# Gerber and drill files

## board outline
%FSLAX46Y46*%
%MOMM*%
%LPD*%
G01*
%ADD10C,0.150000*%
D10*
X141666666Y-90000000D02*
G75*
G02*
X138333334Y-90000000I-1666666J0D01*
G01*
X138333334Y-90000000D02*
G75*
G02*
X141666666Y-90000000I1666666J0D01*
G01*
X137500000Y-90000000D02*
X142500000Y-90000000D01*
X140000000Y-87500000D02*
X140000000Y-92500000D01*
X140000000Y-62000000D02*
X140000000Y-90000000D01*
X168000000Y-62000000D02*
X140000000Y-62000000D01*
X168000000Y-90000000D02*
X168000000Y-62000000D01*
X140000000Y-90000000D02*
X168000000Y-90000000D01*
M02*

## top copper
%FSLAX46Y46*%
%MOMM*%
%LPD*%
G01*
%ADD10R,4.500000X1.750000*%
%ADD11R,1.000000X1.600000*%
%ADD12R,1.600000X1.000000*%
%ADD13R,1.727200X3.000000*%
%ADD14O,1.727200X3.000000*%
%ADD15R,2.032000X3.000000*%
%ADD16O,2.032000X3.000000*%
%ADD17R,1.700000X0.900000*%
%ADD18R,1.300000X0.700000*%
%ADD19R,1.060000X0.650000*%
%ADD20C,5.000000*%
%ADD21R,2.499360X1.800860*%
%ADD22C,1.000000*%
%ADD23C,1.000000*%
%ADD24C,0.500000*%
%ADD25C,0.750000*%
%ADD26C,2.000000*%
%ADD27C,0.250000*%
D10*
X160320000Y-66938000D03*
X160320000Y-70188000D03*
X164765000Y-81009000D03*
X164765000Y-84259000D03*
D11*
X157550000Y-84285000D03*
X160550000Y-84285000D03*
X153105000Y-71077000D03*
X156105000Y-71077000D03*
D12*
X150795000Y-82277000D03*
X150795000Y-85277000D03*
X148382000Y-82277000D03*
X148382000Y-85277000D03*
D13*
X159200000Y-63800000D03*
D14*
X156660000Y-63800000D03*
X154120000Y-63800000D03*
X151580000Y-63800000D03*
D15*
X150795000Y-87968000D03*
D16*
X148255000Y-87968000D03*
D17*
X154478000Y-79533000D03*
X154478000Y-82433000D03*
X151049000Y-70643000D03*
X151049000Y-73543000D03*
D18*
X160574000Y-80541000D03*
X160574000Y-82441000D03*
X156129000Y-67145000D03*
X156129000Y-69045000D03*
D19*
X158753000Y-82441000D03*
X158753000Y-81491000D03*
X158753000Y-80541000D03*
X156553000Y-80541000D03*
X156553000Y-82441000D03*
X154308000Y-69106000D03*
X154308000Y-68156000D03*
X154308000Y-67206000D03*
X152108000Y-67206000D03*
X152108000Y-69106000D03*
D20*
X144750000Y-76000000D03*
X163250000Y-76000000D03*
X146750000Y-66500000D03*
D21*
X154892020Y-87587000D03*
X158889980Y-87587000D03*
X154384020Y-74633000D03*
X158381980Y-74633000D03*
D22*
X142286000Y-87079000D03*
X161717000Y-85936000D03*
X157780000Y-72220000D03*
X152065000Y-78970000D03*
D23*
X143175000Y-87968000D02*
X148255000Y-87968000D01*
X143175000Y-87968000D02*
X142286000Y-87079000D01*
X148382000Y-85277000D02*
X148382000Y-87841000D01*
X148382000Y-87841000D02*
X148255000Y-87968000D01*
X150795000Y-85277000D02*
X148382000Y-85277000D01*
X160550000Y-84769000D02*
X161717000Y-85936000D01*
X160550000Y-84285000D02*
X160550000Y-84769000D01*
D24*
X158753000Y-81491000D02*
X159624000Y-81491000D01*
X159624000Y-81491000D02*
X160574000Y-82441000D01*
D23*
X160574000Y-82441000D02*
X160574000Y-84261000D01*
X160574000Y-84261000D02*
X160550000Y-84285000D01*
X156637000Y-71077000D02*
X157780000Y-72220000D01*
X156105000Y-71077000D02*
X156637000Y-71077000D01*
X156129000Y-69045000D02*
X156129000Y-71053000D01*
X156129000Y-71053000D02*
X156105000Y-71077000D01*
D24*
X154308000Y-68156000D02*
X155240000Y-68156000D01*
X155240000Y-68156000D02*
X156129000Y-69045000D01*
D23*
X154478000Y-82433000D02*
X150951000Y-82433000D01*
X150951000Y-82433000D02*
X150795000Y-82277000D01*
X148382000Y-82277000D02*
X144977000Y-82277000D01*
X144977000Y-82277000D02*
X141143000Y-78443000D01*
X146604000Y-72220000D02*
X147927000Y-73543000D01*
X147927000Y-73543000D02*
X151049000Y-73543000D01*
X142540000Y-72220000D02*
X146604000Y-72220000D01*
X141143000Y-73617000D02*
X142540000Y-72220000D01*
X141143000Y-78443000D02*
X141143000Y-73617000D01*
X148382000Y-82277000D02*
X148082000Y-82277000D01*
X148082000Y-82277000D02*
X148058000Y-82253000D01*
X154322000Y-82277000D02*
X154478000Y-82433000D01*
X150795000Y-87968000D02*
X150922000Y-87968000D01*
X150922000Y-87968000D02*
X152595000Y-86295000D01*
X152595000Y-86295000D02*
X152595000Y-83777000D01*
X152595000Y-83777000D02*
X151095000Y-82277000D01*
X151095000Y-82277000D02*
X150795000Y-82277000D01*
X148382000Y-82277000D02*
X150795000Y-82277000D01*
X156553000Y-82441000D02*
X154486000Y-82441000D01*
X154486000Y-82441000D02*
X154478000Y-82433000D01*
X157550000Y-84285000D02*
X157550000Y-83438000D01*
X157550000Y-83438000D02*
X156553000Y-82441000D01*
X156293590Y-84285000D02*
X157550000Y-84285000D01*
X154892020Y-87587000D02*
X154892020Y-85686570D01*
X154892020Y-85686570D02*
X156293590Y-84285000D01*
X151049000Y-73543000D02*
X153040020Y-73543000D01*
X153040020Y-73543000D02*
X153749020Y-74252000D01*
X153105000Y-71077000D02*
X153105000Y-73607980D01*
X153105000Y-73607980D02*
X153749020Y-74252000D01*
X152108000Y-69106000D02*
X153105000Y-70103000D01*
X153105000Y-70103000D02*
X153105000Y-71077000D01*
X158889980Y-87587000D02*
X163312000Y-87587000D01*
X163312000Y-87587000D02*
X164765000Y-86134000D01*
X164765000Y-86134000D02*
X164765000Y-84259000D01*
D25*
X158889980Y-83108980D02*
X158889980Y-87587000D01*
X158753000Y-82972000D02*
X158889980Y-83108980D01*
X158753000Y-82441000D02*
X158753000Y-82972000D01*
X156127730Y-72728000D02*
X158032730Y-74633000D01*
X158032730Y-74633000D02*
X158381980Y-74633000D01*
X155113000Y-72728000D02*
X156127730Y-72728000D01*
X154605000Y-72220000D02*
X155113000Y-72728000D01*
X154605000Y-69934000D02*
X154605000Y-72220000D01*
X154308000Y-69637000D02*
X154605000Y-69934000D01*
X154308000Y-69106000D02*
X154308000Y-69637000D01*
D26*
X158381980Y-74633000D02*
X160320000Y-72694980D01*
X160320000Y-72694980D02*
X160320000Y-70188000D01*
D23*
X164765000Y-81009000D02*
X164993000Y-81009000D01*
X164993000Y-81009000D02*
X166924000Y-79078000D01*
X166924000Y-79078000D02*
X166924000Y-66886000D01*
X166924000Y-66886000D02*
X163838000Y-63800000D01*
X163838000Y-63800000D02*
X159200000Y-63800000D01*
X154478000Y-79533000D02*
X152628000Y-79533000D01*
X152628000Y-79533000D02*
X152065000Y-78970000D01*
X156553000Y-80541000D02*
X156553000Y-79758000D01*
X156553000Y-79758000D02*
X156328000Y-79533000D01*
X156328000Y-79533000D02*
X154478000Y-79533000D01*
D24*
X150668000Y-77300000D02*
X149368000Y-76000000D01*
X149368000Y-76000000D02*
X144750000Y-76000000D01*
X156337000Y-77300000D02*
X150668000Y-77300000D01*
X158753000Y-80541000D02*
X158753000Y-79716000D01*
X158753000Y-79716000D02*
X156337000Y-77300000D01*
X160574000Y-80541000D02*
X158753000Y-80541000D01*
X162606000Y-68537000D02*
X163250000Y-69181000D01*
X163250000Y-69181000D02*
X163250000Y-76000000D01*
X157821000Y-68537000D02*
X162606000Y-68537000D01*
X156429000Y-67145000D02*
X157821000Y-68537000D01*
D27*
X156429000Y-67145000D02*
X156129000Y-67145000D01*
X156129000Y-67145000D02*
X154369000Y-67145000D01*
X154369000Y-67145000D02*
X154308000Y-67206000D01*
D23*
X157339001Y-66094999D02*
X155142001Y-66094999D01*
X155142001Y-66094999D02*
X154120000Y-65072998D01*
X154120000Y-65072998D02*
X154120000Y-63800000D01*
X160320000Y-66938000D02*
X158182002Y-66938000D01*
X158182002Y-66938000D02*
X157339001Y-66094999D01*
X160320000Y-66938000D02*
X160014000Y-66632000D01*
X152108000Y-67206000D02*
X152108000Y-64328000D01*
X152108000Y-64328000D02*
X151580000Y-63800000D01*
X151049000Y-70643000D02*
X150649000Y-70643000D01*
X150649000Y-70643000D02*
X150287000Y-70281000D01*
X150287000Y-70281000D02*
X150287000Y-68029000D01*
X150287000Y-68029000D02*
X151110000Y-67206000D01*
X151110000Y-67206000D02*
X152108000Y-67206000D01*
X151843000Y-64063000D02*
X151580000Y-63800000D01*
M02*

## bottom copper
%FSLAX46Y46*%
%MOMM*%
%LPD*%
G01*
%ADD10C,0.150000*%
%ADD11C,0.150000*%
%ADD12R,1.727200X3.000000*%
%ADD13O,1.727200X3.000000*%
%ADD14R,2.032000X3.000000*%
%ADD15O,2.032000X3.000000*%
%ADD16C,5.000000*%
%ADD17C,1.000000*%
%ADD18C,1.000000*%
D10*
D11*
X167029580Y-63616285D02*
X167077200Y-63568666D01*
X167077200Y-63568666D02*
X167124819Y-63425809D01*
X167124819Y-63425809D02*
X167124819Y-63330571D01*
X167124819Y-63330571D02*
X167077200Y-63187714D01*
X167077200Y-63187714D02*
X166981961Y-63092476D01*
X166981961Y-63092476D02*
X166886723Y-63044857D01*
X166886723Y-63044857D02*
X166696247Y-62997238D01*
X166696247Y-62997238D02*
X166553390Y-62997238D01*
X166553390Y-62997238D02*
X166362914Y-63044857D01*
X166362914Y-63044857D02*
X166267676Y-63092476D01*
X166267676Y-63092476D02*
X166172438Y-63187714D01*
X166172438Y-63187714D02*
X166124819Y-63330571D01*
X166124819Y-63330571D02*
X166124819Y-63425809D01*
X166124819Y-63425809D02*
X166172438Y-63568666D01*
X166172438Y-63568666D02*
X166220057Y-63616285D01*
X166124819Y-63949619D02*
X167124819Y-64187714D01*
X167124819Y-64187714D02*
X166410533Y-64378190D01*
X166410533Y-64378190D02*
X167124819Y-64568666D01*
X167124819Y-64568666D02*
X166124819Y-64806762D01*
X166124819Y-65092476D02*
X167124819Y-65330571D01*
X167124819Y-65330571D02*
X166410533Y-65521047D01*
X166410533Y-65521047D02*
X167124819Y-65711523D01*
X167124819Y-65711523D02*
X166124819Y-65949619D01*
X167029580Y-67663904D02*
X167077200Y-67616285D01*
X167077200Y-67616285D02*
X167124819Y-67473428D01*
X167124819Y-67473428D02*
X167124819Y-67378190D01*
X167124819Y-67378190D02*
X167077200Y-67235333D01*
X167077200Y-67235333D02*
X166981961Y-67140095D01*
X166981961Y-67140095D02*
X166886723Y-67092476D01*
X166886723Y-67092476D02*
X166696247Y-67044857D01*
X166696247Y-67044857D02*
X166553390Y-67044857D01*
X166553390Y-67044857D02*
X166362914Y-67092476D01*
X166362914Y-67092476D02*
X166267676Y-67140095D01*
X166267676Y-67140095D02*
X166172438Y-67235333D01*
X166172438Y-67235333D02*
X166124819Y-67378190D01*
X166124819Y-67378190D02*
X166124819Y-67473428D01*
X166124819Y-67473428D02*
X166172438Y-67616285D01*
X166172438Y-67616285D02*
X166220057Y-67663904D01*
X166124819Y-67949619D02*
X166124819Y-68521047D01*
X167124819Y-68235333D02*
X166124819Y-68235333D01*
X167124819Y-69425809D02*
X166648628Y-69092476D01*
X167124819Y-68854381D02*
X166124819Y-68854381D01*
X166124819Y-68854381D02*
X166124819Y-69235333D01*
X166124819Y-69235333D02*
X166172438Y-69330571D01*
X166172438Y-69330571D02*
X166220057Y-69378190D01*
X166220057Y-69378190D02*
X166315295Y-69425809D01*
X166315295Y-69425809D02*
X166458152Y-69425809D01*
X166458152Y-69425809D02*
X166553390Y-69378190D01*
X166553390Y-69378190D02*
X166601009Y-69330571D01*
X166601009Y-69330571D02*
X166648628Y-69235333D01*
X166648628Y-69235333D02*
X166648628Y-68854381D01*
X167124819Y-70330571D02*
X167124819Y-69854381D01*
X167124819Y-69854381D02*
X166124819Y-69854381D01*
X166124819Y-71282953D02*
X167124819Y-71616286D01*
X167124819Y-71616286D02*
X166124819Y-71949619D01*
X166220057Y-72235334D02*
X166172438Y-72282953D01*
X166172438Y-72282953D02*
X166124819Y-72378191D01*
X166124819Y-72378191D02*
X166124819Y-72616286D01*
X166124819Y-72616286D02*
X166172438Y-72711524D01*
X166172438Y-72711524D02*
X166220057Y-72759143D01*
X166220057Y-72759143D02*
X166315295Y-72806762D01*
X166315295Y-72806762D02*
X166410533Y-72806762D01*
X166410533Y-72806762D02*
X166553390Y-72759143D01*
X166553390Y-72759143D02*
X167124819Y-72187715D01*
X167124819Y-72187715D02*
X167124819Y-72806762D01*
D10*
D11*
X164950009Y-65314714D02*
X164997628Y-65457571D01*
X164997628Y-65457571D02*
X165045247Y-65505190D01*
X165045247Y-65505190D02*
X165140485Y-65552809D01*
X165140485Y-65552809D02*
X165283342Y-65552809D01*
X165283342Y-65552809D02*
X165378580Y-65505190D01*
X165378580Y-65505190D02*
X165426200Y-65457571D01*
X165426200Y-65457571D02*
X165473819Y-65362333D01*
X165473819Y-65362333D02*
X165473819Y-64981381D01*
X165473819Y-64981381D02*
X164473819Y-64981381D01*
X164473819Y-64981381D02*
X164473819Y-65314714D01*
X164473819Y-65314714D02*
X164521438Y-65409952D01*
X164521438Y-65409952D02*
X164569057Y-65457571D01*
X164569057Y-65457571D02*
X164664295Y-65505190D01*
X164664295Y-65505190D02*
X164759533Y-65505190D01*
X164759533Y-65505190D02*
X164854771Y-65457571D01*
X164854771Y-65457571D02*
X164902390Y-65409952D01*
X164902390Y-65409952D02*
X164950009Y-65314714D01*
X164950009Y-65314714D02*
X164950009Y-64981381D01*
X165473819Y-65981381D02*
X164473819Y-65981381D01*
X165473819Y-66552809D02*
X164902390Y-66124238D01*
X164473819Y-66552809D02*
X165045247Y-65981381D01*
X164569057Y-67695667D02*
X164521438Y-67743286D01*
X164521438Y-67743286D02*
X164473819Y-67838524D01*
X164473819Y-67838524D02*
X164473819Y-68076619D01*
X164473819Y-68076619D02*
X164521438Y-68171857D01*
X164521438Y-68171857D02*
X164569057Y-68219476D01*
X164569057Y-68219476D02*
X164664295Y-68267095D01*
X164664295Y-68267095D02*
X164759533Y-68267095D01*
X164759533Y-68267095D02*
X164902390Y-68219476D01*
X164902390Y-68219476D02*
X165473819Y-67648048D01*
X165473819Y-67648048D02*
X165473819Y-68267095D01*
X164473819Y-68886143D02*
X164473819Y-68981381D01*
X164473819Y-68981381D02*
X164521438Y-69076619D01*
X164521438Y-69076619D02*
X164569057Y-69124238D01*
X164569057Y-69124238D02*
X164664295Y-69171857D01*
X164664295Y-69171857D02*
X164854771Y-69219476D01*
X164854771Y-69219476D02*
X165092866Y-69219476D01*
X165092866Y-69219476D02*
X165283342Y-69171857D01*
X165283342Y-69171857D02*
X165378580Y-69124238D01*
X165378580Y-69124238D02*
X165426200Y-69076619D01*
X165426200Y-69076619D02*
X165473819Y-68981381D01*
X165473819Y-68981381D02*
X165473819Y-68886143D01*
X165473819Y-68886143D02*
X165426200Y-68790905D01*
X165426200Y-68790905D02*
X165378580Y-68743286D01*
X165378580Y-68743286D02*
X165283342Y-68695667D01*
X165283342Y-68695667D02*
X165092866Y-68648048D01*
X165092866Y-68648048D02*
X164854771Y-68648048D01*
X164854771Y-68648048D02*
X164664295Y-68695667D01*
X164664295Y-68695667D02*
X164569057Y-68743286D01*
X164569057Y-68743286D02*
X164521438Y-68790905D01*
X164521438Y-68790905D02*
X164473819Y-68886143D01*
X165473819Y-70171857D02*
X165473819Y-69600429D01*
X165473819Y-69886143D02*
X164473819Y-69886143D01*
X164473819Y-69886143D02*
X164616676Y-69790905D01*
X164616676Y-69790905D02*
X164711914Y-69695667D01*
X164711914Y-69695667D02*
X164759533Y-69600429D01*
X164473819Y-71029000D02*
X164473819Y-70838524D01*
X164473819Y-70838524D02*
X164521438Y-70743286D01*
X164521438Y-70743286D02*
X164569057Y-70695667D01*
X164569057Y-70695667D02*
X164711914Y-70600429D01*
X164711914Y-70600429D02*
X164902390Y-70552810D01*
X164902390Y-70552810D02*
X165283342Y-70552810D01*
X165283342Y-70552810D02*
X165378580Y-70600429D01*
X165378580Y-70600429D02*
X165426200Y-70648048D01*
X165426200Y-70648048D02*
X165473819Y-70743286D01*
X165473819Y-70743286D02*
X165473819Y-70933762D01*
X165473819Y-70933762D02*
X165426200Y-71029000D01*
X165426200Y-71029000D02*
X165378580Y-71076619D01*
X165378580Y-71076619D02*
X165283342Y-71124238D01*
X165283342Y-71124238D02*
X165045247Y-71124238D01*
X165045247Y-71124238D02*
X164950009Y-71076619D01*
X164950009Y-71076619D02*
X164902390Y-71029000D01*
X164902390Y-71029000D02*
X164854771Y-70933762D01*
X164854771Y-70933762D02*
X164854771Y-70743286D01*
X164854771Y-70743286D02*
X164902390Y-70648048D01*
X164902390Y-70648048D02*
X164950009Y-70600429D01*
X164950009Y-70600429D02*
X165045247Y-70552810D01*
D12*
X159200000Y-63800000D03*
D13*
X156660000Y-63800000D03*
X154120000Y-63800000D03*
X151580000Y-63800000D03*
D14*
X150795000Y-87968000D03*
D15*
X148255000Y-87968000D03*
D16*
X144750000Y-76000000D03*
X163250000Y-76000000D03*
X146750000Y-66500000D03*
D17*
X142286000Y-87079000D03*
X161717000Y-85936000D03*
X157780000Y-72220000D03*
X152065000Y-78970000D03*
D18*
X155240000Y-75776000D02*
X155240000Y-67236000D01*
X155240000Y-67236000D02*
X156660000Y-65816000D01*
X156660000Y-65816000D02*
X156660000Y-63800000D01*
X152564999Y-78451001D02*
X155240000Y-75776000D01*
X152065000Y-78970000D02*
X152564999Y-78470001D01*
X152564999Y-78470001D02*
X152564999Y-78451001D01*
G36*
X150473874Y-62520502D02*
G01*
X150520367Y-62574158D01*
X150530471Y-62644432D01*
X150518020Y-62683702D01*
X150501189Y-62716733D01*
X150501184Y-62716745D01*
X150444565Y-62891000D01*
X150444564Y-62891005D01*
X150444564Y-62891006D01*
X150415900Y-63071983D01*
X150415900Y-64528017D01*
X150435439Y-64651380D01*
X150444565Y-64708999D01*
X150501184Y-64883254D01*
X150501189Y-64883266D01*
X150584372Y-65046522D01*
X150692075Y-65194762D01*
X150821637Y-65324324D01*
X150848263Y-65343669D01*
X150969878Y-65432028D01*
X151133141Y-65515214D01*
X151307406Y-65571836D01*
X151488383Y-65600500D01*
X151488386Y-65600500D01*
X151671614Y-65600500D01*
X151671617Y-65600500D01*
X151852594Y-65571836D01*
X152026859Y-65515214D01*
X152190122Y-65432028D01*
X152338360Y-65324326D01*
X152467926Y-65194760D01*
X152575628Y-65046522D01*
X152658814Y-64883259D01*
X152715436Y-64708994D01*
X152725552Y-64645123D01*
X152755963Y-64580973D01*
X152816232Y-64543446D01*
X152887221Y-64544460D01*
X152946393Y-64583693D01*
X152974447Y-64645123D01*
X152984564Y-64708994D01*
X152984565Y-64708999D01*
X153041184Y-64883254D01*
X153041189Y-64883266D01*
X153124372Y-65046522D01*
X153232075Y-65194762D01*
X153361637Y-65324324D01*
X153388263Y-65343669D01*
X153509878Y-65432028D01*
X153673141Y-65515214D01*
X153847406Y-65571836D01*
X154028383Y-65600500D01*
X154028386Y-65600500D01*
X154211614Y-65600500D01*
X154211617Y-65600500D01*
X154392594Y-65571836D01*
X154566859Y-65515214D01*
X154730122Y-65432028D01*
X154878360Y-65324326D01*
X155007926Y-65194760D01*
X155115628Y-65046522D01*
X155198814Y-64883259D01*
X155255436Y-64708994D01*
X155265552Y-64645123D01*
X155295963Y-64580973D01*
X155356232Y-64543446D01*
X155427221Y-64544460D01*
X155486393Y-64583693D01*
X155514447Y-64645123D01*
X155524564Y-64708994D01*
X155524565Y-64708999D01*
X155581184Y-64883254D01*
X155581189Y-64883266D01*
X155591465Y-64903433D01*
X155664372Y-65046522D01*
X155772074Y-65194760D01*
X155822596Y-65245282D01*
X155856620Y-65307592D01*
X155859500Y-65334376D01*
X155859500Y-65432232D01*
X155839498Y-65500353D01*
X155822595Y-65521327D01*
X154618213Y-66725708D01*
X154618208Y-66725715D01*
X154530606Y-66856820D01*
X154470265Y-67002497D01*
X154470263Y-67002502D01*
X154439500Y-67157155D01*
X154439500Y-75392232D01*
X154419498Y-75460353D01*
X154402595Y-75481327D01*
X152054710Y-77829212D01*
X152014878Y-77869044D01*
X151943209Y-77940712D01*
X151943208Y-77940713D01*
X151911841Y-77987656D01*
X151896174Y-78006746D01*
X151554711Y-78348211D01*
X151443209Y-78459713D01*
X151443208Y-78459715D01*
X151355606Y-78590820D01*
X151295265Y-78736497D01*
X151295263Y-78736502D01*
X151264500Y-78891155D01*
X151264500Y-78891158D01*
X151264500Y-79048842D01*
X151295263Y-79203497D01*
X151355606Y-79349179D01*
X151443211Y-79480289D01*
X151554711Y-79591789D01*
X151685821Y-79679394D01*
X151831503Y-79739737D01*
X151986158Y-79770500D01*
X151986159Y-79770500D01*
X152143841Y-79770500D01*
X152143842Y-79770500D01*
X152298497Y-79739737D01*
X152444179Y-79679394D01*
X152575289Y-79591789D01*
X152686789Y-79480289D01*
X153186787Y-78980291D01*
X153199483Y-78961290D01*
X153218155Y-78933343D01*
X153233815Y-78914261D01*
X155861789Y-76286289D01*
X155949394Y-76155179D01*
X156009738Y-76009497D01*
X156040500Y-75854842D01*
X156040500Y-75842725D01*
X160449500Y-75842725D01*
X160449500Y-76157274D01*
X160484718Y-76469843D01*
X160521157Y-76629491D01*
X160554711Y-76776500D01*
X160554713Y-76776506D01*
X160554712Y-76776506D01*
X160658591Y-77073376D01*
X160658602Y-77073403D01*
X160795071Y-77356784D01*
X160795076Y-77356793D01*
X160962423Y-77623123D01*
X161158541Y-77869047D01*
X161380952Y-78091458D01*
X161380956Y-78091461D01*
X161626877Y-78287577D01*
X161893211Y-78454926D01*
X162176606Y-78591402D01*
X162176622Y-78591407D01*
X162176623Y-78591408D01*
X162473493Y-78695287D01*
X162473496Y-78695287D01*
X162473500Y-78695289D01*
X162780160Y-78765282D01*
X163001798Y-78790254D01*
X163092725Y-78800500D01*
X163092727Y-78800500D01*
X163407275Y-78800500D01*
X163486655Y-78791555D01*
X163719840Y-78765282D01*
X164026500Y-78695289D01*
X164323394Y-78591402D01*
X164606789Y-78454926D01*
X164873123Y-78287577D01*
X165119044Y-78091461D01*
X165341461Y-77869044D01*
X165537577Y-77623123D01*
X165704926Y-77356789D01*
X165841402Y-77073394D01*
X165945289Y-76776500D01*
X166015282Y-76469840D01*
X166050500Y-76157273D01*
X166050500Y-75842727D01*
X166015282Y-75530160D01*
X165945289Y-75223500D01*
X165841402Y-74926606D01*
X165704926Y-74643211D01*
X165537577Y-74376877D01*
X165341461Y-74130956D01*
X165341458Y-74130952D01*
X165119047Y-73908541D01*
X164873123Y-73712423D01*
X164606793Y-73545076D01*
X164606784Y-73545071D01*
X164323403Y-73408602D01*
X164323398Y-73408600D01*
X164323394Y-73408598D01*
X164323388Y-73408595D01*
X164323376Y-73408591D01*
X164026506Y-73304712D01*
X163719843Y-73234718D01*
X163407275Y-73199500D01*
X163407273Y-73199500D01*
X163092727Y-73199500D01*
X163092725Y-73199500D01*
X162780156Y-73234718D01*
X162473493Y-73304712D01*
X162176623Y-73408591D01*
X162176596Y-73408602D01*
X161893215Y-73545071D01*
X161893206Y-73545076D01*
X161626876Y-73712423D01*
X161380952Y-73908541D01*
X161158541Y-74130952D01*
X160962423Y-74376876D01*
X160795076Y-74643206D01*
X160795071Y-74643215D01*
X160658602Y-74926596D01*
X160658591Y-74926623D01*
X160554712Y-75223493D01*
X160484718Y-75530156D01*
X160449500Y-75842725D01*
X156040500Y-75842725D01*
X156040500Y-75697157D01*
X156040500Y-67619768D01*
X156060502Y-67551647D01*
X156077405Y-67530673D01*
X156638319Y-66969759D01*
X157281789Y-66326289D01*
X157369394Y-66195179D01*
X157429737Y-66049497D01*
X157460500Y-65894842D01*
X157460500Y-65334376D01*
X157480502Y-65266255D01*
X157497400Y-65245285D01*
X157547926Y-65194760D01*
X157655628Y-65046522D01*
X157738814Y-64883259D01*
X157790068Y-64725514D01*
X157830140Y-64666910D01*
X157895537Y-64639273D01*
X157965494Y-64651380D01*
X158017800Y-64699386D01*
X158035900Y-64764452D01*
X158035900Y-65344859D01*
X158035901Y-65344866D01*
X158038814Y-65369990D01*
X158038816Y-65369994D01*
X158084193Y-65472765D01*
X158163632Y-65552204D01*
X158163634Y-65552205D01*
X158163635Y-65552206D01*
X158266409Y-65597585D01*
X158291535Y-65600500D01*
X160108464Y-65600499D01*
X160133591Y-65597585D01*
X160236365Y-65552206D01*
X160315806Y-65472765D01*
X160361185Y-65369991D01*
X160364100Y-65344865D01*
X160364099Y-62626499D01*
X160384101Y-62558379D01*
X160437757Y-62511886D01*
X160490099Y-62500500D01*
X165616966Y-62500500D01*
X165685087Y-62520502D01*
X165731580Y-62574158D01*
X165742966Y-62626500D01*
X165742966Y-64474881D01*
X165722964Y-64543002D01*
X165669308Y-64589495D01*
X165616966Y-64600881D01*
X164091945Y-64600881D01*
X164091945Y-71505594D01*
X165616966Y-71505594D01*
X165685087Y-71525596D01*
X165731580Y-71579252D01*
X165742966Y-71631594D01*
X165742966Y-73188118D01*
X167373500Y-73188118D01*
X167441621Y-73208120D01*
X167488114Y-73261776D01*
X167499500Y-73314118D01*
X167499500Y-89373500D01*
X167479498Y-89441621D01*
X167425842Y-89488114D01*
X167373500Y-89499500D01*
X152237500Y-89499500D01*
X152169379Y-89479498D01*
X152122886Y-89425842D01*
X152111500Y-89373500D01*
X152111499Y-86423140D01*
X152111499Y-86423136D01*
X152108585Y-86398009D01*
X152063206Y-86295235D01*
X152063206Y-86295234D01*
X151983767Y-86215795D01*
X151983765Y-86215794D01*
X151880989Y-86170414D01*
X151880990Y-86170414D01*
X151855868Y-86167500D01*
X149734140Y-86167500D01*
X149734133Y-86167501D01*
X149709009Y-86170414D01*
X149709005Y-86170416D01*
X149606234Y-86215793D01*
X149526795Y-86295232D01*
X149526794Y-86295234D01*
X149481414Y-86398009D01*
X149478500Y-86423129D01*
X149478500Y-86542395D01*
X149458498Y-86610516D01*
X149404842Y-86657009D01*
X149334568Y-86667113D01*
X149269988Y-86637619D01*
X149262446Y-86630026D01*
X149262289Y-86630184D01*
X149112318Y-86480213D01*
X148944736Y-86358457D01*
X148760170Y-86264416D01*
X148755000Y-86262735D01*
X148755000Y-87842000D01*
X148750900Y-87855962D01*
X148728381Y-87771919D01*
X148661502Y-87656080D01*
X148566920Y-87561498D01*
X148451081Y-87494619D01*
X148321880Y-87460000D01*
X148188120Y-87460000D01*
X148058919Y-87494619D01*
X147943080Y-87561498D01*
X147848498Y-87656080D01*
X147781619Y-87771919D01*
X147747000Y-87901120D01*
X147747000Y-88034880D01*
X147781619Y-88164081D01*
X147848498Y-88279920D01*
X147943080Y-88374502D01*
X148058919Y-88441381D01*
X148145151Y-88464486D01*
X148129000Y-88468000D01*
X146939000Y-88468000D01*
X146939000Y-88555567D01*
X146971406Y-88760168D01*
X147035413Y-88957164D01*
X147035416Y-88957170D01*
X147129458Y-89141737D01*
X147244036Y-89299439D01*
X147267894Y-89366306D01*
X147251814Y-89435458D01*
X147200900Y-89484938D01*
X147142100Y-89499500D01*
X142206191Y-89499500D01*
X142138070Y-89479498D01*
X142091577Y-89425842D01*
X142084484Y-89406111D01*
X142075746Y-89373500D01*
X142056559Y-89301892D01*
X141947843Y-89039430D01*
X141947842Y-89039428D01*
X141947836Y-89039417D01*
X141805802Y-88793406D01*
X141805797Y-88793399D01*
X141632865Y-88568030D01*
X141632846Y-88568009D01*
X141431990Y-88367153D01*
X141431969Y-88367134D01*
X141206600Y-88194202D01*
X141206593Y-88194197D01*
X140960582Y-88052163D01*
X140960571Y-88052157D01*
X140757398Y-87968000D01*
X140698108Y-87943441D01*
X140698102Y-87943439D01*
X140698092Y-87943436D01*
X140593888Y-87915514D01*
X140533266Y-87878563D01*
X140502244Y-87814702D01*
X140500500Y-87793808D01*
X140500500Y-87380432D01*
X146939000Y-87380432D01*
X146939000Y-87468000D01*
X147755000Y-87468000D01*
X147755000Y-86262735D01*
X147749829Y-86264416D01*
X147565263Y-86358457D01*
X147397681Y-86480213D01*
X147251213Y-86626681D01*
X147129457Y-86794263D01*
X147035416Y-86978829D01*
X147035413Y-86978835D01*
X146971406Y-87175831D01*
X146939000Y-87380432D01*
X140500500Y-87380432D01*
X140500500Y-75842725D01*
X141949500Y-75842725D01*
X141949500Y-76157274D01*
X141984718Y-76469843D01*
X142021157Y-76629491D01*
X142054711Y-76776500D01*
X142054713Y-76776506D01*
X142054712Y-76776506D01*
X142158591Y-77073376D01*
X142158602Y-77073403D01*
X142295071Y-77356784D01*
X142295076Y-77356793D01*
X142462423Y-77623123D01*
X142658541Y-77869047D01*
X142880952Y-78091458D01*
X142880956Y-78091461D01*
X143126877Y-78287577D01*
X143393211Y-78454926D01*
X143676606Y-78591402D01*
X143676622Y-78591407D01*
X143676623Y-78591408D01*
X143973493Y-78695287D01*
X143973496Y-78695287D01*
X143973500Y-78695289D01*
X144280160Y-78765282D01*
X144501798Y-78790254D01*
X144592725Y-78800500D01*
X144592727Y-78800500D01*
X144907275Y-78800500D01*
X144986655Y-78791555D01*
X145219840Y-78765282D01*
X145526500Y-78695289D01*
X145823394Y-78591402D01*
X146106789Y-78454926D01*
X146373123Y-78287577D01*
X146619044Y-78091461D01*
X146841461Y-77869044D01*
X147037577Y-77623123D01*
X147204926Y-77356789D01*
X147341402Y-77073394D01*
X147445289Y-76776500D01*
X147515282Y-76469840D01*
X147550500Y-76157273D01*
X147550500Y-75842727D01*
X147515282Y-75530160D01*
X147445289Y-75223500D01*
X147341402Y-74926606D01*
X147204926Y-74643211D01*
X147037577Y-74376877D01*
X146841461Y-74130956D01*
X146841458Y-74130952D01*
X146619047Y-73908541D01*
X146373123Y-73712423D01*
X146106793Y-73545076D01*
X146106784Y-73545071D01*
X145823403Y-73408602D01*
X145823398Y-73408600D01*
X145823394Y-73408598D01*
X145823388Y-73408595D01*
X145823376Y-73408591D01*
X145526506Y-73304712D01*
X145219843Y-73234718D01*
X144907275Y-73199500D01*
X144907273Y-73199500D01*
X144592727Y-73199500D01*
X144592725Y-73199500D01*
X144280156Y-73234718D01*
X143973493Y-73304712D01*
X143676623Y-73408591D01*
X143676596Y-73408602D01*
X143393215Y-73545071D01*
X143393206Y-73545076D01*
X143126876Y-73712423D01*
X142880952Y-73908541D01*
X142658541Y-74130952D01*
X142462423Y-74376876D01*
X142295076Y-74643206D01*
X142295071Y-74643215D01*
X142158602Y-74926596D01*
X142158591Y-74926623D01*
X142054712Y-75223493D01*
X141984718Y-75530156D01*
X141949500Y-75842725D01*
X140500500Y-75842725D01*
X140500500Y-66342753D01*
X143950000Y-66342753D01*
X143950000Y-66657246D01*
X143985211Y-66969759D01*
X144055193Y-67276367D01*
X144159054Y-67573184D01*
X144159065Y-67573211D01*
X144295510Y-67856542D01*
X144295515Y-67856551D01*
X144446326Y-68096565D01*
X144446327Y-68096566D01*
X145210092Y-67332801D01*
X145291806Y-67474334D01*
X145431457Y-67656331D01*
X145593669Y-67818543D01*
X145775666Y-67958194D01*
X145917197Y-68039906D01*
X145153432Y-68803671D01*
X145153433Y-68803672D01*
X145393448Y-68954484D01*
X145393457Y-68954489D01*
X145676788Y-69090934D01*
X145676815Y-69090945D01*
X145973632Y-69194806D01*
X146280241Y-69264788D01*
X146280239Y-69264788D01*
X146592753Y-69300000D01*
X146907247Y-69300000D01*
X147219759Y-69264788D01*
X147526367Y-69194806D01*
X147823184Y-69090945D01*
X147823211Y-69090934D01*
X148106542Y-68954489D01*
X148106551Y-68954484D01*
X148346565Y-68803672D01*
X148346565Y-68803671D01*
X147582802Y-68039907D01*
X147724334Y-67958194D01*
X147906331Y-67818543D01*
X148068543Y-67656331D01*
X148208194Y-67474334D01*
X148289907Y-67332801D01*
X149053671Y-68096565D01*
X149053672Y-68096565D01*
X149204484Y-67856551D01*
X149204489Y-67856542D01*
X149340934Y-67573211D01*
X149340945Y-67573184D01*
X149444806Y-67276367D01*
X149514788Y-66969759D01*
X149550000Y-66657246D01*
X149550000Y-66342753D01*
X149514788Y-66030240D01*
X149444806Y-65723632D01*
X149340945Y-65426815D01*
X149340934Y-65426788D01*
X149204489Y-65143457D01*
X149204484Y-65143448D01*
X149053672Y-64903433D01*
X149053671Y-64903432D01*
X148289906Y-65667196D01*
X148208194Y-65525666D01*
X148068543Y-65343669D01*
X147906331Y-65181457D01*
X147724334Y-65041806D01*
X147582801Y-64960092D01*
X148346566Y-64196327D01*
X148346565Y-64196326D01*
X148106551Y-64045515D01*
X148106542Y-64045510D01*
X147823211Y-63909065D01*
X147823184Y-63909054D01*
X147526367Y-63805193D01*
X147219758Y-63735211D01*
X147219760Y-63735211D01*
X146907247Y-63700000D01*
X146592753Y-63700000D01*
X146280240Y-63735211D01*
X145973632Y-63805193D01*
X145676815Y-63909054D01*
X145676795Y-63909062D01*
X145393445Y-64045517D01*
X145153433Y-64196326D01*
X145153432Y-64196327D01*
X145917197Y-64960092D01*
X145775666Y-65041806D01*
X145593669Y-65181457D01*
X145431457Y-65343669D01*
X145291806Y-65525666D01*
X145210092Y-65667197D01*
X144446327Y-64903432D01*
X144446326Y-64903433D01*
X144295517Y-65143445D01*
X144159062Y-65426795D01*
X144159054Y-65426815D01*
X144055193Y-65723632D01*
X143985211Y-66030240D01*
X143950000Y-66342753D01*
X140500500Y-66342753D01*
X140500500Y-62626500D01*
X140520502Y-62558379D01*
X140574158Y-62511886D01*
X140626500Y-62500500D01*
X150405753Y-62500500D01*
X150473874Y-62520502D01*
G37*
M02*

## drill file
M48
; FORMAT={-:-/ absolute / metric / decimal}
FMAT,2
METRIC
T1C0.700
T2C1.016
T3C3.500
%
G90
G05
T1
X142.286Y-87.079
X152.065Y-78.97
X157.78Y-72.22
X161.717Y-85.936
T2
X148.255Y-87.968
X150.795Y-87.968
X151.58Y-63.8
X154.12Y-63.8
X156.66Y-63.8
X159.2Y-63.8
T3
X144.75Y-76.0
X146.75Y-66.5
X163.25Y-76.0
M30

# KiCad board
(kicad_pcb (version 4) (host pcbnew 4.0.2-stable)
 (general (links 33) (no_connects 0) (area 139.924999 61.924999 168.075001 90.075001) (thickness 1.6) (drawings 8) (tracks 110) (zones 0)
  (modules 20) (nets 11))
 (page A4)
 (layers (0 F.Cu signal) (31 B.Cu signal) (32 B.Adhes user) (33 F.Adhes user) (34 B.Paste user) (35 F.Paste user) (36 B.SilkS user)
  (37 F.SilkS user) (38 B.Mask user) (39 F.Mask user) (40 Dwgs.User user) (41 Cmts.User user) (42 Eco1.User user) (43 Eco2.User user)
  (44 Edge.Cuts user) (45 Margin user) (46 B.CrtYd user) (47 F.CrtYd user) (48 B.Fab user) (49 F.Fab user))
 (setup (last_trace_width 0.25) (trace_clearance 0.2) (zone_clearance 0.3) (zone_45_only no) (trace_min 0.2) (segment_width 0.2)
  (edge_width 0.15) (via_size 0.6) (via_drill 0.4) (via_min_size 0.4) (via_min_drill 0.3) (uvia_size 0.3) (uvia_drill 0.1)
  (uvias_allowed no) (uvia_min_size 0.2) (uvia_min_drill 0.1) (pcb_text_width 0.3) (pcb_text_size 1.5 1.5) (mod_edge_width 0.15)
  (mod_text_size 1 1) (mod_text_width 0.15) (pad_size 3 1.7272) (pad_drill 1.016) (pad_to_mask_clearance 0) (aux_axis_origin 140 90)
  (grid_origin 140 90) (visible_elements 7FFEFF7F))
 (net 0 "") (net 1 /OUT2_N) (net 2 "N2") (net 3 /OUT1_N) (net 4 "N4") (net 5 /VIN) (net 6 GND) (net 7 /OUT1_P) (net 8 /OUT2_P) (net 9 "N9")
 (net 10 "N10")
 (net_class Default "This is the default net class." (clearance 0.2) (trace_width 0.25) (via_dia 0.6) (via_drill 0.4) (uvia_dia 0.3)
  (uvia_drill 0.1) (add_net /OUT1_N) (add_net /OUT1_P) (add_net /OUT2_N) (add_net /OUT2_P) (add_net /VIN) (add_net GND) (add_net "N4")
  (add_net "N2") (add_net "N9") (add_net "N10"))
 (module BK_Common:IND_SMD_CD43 (layer F.Cu) (at 160.32 68.563 270)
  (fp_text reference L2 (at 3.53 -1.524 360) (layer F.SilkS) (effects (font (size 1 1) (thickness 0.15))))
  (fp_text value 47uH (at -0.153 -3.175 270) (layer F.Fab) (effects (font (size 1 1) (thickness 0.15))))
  (pad 1 smd rect (at -1.625 0 270) (size 1.75 4.5) (layers F.Cu F.Paste F.Mask) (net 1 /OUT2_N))
  (pad 2 smd rect (at 1.625 0 270) (size 1.75 4.5) (layers F.Cu F.Paste F.Mask) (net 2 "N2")))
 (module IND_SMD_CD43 (layer F.Cu) (at 164.765 82.634 270)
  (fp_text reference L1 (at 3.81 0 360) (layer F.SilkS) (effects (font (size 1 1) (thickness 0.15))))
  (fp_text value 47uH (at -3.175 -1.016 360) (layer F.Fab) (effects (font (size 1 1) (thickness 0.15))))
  (pad 1 smd rect (at -1.625 0 270) (size 1.75 4.5) (layers F.Cu F.Paste F.Mask) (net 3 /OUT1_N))
  (pad 2 smd rect (at 1.625 0 270) (size 1.75 4.5) (layers F.Cu F.Paste F.Mask) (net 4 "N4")))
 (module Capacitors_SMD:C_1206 (layer F.Cu) (at 159.05 84.285)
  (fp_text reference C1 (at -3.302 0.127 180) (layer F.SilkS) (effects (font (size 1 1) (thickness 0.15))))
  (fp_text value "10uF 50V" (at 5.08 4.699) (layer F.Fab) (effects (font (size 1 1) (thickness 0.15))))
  (pad 1 smd rect (at -1.5 0) (size 1 1.6) (layers F.Cu F.Paste F.Mask) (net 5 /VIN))
  (pad 2 smd rect (at 1.5 0) (size 1 1.6) (layers F.Cu F.Paste F.Mask) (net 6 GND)))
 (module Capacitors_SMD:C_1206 (layer F.Cu) (at 154.605 71.077)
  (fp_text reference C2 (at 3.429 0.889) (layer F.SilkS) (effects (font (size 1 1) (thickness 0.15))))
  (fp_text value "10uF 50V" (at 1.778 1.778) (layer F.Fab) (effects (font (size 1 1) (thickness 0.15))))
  (pad 1 smd rect (at -1.5 0) (size 1 1.6) (layers F.Cu F.Paste F.Mask) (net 5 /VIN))
  (pad 2 smd rect (at 1.5 0) (size 1 1.6) (layers F.Cu F.Paste F.Mask) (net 6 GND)))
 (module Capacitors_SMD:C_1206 (layer F.Cu) (at 150.795 83.777 270)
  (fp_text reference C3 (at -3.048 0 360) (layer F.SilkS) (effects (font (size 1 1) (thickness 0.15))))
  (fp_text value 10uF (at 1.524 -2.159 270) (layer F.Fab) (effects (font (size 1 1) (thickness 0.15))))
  (pad 1 smd rect (at -1.5 0 270) (size 1 1.6) (layers F.Cu F.Paste F.Mask) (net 5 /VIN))
  (pad 2 smd rect (at 1.5 0 270) (size 1 1.6) (layers F.Cu F.Paste F.Mask) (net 6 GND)))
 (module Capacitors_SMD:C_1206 (layer F.Cu) (at 148.382 83.777 270)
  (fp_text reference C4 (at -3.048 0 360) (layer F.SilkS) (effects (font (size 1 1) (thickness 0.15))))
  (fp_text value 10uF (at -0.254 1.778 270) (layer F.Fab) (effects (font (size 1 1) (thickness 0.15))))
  (pad 1 smd rect (at -1.5 0 270) (size 1 1.6) (layers F.Cu F.Paste F.Mask) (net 5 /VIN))
  (pad 2 smd rect (at 1.5 0 270) (size 1 1.6) (layers F.Cu F.Paste F.Mask) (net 6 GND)))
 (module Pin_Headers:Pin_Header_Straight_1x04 (layer F.Cu) (at 159.2 63.8 270)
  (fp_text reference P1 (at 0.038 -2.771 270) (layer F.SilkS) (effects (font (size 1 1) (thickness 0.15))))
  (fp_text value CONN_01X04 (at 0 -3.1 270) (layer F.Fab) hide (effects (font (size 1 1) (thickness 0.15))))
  (pad 1 thru_hole rect (at 0 0 270) (size 3 1.7272) (drill 1.016) (layers *.Cu *.Mask F.SilkS) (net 3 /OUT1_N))
  (pad 2 thru_hole oval (at 0 2.54 270) (size 3 1.7272) (drill 1.016) (layers *.Cu *.Mask F.SilkS) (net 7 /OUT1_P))
  (pad 3 thru_hole oval (at 0 5.08 270) (size 3 1.7272) (drill 1.016) (layers *.Cu *.Mask F.SilkS) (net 1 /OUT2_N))
  (pad 4 thru_hole oval (at 0 7.62 270) (size 3 1.7272) (drill 1.016) (layers *.Cu *.Mask F.SilkS) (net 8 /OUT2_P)))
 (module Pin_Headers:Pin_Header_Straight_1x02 (layer F.Cu) (at 150.795 87.968 270)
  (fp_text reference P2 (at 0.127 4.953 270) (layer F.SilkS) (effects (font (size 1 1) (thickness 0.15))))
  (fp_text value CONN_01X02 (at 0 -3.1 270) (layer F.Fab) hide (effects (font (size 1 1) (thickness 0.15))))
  (pad 1 thru_hole rect (at 0 0 270) (size 3 2.032) (drill 1.016) (layers *.Cu *.Mask F.SilkS) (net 5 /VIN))
  (pad 2 thru_hole oval (at 0 2.54 270) (size 3 2.032) (drill 1.016) (layers *.Cu *.Mask F.SilkS) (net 6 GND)))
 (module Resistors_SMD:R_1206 (layer F.Cu) (at 154.478 80.983 270)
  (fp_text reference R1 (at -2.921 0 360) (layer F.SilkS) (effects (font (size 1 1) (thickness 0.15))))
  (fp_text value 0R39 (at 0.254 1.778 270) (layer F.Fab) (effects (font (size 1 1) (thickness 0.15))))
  (pad 1 smd rect (at -1.45 0 270) (size 0.9 1.7) (layers F.Cu F.Paste F.Mask) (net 7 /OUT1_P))
  (pad 2 smd rect (at 1.45 0 270) (size 0.9 1.7) (layers F.Cu F.Paste F.Mask) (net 5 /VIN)))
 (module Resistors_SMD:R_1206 (layer F.Cu) (at 151.049 72.093 270)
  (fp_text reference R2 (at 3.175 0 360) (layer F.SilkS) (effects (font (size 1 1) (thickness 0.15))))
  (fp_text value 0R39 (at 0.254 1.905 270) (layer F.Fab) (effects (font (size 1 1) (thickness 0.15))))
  (pad 1 smd rect (at -1.45 0 270) (size 0.9 1.7) (layers F.Cu F.Paste F.Mask) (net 8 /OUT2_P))
  (pad 2 smd rect (at 1.45 0 270) (size 0.9 1.7) (layers F.Cu F.Paste F.Mask) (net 5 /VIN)))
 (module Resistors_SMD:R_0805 (layer F.Cu) (at 160.574 81.491 270)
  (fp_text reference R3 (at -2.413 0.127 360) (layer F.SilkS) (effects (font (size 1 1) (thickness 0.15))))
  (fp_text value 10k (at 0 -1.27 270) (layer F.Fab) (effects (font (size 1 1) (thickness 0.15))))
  (pad 1 smd rect (at -0.95 0 270) (size 0.7 1.3) (layers F.Cu F.Paste F.Mask) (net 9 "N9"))
  (pad 2 smd rect (at 0.95 0 270) (size 0.7 1.3) (layers F.Cu F.Paste F.Mask) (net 6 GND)))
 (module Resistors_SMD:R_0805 (layer F.Cu) (at 156.129 68.095 270)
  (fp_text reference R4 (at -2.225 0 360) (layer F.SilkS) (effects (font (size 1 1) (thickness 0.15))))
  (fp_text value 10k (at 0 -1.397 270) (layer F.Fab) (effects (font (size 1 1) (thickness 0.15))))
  (pad 1 smd rect (at -0.95 0 270) (size 0.7 1.3) (layers F.Cu F.Paste F.Mask) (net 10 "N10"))
  (pad 2 smd rect (at 0.95 0 270) (size 0.7 1.3) (layers F.Cu F.Paste F.Mask) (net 6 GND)))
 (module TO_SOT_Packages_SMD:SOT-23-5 (layer F.Cu) (at 157.653 81.491 180)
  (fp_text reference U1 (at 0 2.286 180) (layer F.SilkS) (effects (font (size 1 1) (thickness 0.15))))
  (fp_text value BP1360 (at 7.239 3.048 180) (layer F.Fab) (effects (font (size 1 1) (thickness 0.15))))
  (pad 1 smd rect (at -1.1 -0.95 180) (size 1.06 0.65) (layers F.Cu F.Paste F.Mask) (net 4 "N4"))
  (pad 2 smd rect (at -1.1 0 180) (size 1.06 0.65) (layers F.Cu F.Paste F.Mask) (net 6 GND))
  (pad 3 smd rect (at -1.1 0.95 180) (size 1.06 0.65) (layers F.Cu F.Paste F.Mask) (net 9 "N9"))
  (pad 4 smd rect (at 1.1 0.95 180) (size 1.06 0.65) (layers F.Cu F.Paste F.Mask) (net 7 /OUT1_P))
  (pad 5 smd rect (at 1.1 -0.95 180) (size 1.06 0.65) (layers F.Cu F.Paste F.Mask) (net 5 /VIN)))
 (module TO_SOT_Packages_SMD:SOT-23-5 (layer F.Cu) (at 153.208 68.156 180)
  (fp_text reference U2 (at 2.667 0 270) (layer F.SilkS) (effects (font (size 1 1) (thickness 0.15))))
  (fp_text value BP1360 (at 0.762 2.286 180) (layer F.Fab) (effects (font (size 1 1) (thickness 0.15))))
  (pad 1 smd rect (at -1.1 -0.95 180) (size 1.06 0.65) (layers F.Cu F.Paste F.Mask) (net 2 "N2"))
  (pad 2 smd rect (at -1.1 0 180) (size 1.06 0.65) (layers F.Cu F.Paste F.Mask) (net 6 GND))
  (pad 3 smd rect (at -1.1 0.95 180) (size 1.06 0.65) (layers F.Cu F.Paste F.Mask) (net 10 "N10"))
  (pad 4 smd rect (at 1.1 0.95 180) (size 1.06 0.65) (layers F.Cu F.Paste F.Mask) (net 8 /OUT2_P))
  (pad 5 smd rect (at 1.1 -0.95 180) (size 1.06 0.65) (layers F.Cu F.Paste F.Mask) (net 5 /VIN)))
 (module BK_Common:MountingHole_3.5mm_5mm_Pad (layer F.Cu) (at 144.75 76)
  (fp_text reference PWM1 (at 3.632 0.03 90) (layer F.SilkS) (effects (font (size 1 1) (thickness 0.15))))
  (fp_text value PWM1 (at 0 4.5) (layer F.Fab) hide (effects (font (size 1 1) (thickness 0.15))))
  (pad 1 thru_hole circle (at 0 0) (size 5 5) (drill 3.5) (layers *.Cu *.Mask F.SilkS) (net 9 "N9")))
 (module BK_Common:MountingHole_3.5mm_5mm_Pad (layer F.Cu) (at 163.25 76)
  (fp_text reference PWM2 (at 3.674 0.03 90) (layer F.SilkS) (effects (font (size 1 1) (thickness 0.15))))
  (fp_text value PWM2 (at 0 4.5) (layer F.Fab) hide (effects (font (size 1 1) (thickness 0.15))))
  (pad 1 thru_hole circle (at 0 0) (size 5 5) (drill 3.5) (layers *.Cu *.Mask F.SilkS) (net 10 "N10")))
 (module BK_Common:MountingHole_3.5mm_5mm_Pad (layer F.Cu) (at 146.75 66.5)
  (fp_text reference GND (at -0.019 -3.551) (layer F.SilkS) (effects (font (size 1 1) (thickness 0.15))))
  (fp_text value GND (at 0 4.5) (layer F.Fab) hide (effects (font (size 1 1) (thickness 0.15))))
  (pad 1 thru_hole circle (at 0 0) (size 5 5) (drill 3.5) (layers *.Cu *.Mask F.SilkS) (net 6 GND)))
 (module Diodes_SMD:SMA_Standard (layer F.Cu) (at 156.891 87.587)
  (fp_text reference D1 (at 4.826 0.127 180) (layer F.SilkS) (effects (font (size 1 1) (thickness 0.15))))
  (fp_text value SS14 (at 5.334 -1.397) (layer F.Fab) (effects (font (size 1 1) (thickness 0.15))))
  (pad 1 smd rect (at -1.99898 0) (size 2.49936 1.80086) (layers F.Cu F.Paste F.Mask) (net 5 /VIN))
  (pad 2 smd rect (at 1.99898 0) (size 2.49936 1.80086) (layers F.Cu F.Paste F.Mask) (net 4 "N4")))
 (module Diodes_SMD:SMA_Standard (layer F.Cu) (at 156.383 74.633)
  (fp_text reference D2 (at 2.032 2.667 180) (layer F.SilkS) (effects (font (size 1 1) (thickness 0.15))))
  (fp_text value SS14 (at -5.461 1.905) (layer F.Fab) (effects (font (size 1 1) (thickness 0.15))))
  (pad 1 smd rect (at -1.99898 0) (size 2.49936 1.80086) (layers F.Cu F.Paste F.Mask) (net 5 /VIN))
  (pad 2 smd rect (at 1.99898 0) (size 2.49936 1.80086) (layers F.Cu F.Paste F.Mask) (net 2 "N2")))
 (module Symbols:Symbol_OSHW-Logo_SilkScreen (layer F.Cu) (at 143.556 81.999)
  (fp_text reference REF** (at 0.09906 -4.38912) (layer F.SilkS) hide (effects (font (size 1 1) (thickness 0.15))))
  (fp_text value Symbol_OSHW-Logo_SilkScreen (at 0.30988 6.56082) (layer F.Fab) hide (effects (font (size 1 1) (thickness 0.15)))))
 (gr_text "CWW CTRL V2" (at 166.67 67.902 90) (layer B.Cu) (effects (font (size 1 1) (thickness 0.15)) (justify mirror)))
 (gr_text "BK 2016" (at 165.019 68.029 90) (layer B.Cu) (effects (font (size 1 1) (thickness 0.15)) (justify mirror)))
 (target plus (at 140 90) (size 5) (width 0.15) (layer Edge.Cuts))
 (gr_line (start 140 62) (end 140 90) (layer Edge.Cuts) (width 0.15))
 (gr_line (start 168 62) (end 140 62) (layer Edge.Cuts) (width 0.15))
 (gr_line (start 168 90) (end 168 62) (layer Edge.Cuts) (width 0.15))
 (gr_line (start 140 90) (end 168 90) (layer Edge.Cuts) (width 0.15))
 (segment (start 143.175 87.968) (end 148.255 87.968) (width 1) (layer F.Cu) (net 6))
 (via (at 142.286 87.079) (size 1) (drill 0.7) (layers F.Cu B.Cu) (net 6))
 (segment (start 143.175 87.968) (end 142.286 87.079) (width 1) (layer F.Cu) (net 6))
 (segment (start 148.382 85.277) (end 148.382 87.841) (width 1) (layer F.Cu) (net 6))
 (segment (start 148.382 87.841) (end 148.255 87.968) (width 1) (layer F.Cu) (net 6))
 (segment (start 150.795 85.277) (end 148.382 85.277) (width 1) (layer F.Cu) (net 6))
 (via (at 161.717 85.936) (size 1) (drill 0.7) (layers F.Cu B.Cu) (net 6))
 (segment (start 160.55 84.769) (end 161.717 85.936) (width 1) (layer F.Cu) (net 6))
 (segment (start 160.55 84.285) (end 160.55 84.769) (width 1) (layer F.Cu) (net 6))
 (segment (start 158.753 81.491) (end 159.624 81.491) (width 0.5) (layer F.Cu) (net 6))
 (segment (start 159.624 81.491) (end 160.574 82.441) (width 0.5) (layer F.Cu) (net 6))
 (segment (start 160.574 82.441) (end 160.574 84.261) (width 1) (layer F.Cu) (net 6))
 (segment (start 160.574 84.261) (end 160.55 84.285) (width 1) (layer F.Cu) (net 6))
 (via (at 157.78 72.22) (size 1) (drill 0.7) (layers F.Cu B.Cu) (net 6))
 (segment (start 156.637 71.077) (end 157.78 72.22) (width 1) (layer F.Cu) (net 6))
 (segment (start 156.105 71.077) (end 156.637 71.077) (width 1) (layer F.Cu) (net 6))
 (segment (start 156.129 69.045) (end 156.129 71.053) (width 1) (layer F.Cu) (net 6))
 (segment (start 156.129 71.053) (end 156.105 71.077) (width 1) (layer F.Cu) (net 6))
 (segment (start 154.308 68.156) (end 155.24 68.156) (width 0.5) (layer F.Cu) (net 6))
 (segment (start 155.24 68.156) (end 156.129 69.045) (width 0.5) (layer F.Cu) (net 6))
 (segment (start 154.478 82.433) (end 150.951 82.433) (width 1) (layer F.Cu) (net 5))
 (segment (start 150.951 82.433) (end 150.795 82.277) (width 1) (layer F.Cu) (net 5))
 (segment (start 148.382 82.277) (end 144.977 82.277) (width 1) (layer F.Cu) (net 5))
 (segment (start 144.977 82.277) (end 141.143 78.443) (width 1) (layer F.Cu) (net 5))
 (segment (start 146.604 72.22) (end 147.927 73.543) (width 1) (layer F.Cu) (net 5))
 (segment (start 147.927 73.543) (end 151.049 73.543) (width 1) (layer F.Cu) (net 5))
 (segment (start 142.54 72.22) (end 146.604 72.22) (width 1) (layer F.Cu) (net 5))
 (segment (start 141.143 73.617) (end 142.54 72.22) (width 1) (layer F.Cu) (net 5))
 (segment (start 141.143 78.443) (end 141.143 73.617) (width 1) (layer F.Cu) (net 5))
 (segment (start 148.382 82.277) (end 148.082 82.277) (width 1) (layer F.Cu) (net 5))
 (segment (start 148.082 82.277) (end 148.058 82.253) (width 1) (layer F.Cu) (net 5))
 (segment (start 154.322 82.277) (end 154.478 82.433) (width 1) (layer F.Cu) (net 5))
 (segment (start 150.795 87.968) (end 150.922 87.968) (width 1) (layer F.Cu) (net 5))
 (segment (start 150.922 87.968) (end 152.595 86.295) (width 1) (layer F.Cu) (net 5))
 (segment (start 152.595 86.295) (end 152.595 83.777) (width 1) (layer F.Cu) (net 5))
 (segment (start 152.595 83.777) (end 151.095 82.277) (width 1) (layer F.Cu) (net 5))
 (segment (start 151.095 82.277) (end 150.795 82.277) (width 1) (layer F.Cu) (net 5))
 (segment (start 148.382 82.277) (end 150.795 82.277) (width 1) (layer F.Cu) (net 5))
 (segment (start 156.553 82.441) (end 154.486 82.441) (width 1) (layer F.Cu) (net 5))
 (segment (start 154.486 82.441) (end 154.478 82.433) (width 1) (layer F.Cu) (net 5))
 (segment (start 157.55 84.285) (end 157.55 83.438) (width 1) (layer F.Cu) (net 5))
 (segment (start 157.55 83.438) (end 156.553 82.441) (width 1) (layer F.Cu) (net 5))
 (segment (start 156.29359 84.285) (end 157.55 84.285) (width 1) (layer F.Cu) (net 5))
 (segment (start 154.89202 87.587) (end 154.89202 85.68657) (width 1) (layer F.Cu) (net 5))
 (segment (start 154.89202 85.68657) (end 156.29359 84.285) (width 1) (layer F.Cu) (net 5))
 (segment (start 151.049 73.543) (end 153.04002 73.543) (width 1) (layer F.Cu) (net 5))
 (segment (start 153.04002 73.543) (end 153.74902 74.252) (width 1) (layer F.Cu) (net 5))
 (segment (start 153.105 71.077) (end 153.105 73.60798) (width 1) (layer F.Cu) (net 5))
 (segment (start 153.105 73.60798) (end 153.74902 74.252) (width 1) (layer F.Cu) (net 5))
 (segment (start 152.108 69.106) (end 153.105 70.103) (width 1) (layer F.Cu) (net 5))
 (segment (start 153.105 70.103) (end 153.105 71.077) (width 1) (layer F.Cu) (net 5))
 (segment (start 158.88998 87.587) (end 163.312 87.587) (width 1) (layer F.Cu) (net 4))
 (segment (start 163.312 87.587) (end 164.765 86.134) (width 1) (layer F.Cu) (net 4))
 (segment (start 164.765 86.134) (end 164.765 84.259) (width 1) (layer F.Cu) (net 4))
 (segment (start 158.88998 83.10898) (end 158.88998 87.587) (width 0.75) (layer F.Cu) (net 4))
 (segment (start 158.753 82.972) (end 158.88998 83.10898) (width 0.75) (layer F.Cu) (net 4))
 (segment (start 158.753 82.441) (end 158.753 82.972) (width 0.75) (layer F.Cu) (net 4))
 (segment (start 156.12773 72.728) (end 158.03273 74.633) (width 0.75) (layer F.Cu) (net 2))
 (segment (start 158.03273 74.633) (end 158.38198 74.633) (width 0.75) (layer F.Cu) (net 2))
 (segment (start 155.113 72.728) (end 156.12773 72.728) (width 0.75) (layer F.Cu) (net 2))
 (segment (start 154.605 72.22) (end 155.113 72.728) (width 0.75) (layer F.Cu) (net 2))
 (segment (start 154.605 69.934) (end 154.605 72.22) (width 0.75) (layer F.Cu) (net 2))
 (segment (start 154.308 69.637) (end 154.605 69.934) (width 0.75) (layer F.Cu) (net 2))
 (segment (start 154.308 69.106) (end 154.308 69.637) (width 0.75) (layer F.Cu) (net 2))
 (segment (start 158.38198 74.633) (end 160.32 72.69498) (width 2) (layer F.Cu) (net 2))
 (segment (start 160.32 72.69498) (end 160.32 70.188) (width 2) (layer F.Cu) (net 2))
 (segment (start 164.765 81.009) (end 164.993 81.009) (width 1) (layer F.Cu) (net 3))
 (segment (start 164.993 81.009) (end 166.924 79.078) (width 1) (layer F.Cu) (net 3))
 (segment (start 166.924 79.078) (end 166.924 66.886) (width 1) (layer F.Cu) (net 3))
 (segment (start 166.924 66.886) (end 163.838 63.8) (width 1) (layer F.Cu) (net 3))
 (segment (start 163.838 63.8) (end 159.2 63.8) (width 1) (layer F.Cu) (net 3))
 (segment (start 155.24 75.776) (end 155.24 67.236) (width 1) (layer B.Cu) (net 7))
 (segment (start 155.24 67.236) (end 156.66 65.816) (width 1) (layer B.Cu) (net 7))
 (segment (start 156.66 65.816) (end 156.66 63.8) (width 1) (layer B.Cu) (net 7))
 (segment (start 152.564999 78.451001) (end 155.24 75.776) (width 1) (layer B.Cu) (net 7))
 (segment (start 152.065 78.97) (end 152.564999 78.470001) (width 1) (layer B.Cu) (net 7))
 (segment (start 152.564999 78.470001) (end 152.564999 78.451001) (width 1) (layer B.Cu) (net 7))
 (via (at 152.065 78.97) (size 1) (drill 0.7) (layers F.Cu B.Cu) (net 7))
 (segment (start 154.478 79.533) (end 152.628 79.533) (width 1) (layer F.Cu) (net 7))
 (segment (start 152.628 79.533) (end 152.065 78.97) (width 1) (layer F.Cu) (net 7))
 (segment (start 156.553 80.541) (end 156.553 79.758) (width 1) (layer F.Cu) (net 7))
 (segment (start 156.553 79.758) (end 156.328 79.533) (width 1) (layer F.Cu) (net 7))
 (segment (start 156.328 79.533) (end 154.478 79.533) (width 1) (layer F.Cu) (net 7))
 (segment (start 150.668 77.3) (end 149.368 76) (width 0.5) (layer F.Cu) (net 9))
 (segment (start 149.368 76) (end 144.75 76) (width 0.5) (layer F.Cu) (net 9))
 (segment (start 156.337 77.3) (end 150.668 77.3) (width 0.5) (layer F.Cu) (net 9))
 (segment (start 158.753 80.541) (end 158.753 79.716) (width 0.5) (layer F.Cu) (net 9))
 (segment (start 158.753 79.716) (end 156.337 77.3) (width 0.5) (layer F.Cu) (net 9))
 (segment (start 160.574 80.541) (end 158.753 80.541) (width 0.5) (layer F.Cu) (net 9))
 (segment (start 162.606 68.537) (end 163.25 69.181) (width 0.5) (layer F.Cu) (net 10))
 (segment (start 163.25 69.181) (end 163.25 76) (width 0.5) (layer F.Cu) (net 10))
 (segment (start 157.821 68.537) (end 162.606 68.537) (width 0.5) (layer F.Cu) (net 10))
 (segment (start 156.429 67.145) (end 157.821 68.537) (width 0.5) (layer F.Cu) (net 10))
 (segment (start 156.429 67.145) (end 156.129 67.145) (width 0.25) (layer F.Cu) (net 10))
 (segment (start 156.129 67.145) (end 154.369 67.145) (width 0.25) (layer F.Cu) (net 10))
 (segment (start 154.369 67.145) (end 154.308 67.206) (width 0.25) (layer F.Cu) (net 10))
 (segment (start 157.339001 66.094999) (end 155.142001 66.094999) (width 1) (layer F.Cu) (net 1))
 (segment (start 155.142001 66.094999) (end 154.12 65.072998) (width 1) (layer F.Cu) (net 1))
 (segment (start 154.12 65.072998) (end 154.12 63.8) (width 1) (layer F.Cu) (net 1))
 (segment (start 160.32 66.938) (end 158.182002 66.938) (width 1) (layer F.Cu) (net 1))
 (segment (start 158.182002 66.938) (end 157.339001 66.094999) (width 1) (layer F.Cu) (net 1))
 (segment (start 160.32 66.938) (end 160.014 66.632) (width 1) (layer F.Cu) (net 1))
 (segment (start 152.108 67.206) (end 152.108 64.328) (width 1) (layer F.Cu) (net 8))
 (segment (start 152.108 64.328) (end 151.58 63.8) (width 1) (layer F.Cu) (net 8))
 (segment (start 151.049 70.643) (end 150.649 70.643) (width 1) (layer F.Cu) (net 8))
 (segment (start 150.649 70.643) (end 150.287 70.281) (width 1) (layer F.Cu) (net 8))
 (segment (start 150.287 70.281) (end 150.287 68.029) (width 1) (layer F.Cu) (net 8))
 (segment (start 150.287 68.029) (end 151.11 67.206) (width 1) (layer F.Cu) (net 8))
 (segment (start 151.11 67.206) (end 152.108 67.206) (width 1) (layer F.Cu) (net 8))
 (segment (start 151.843 64.063) (end 151.58 63.8) (width 1) (layer F.Cu) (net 8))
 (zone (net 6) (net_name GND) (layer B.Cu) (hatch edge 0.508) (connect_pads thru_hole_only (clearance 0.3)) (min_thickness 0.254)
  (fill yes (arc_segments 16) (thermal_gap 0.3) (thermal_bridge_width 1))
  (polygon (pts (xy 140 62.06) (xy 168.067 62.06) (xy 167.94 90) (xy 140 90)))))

